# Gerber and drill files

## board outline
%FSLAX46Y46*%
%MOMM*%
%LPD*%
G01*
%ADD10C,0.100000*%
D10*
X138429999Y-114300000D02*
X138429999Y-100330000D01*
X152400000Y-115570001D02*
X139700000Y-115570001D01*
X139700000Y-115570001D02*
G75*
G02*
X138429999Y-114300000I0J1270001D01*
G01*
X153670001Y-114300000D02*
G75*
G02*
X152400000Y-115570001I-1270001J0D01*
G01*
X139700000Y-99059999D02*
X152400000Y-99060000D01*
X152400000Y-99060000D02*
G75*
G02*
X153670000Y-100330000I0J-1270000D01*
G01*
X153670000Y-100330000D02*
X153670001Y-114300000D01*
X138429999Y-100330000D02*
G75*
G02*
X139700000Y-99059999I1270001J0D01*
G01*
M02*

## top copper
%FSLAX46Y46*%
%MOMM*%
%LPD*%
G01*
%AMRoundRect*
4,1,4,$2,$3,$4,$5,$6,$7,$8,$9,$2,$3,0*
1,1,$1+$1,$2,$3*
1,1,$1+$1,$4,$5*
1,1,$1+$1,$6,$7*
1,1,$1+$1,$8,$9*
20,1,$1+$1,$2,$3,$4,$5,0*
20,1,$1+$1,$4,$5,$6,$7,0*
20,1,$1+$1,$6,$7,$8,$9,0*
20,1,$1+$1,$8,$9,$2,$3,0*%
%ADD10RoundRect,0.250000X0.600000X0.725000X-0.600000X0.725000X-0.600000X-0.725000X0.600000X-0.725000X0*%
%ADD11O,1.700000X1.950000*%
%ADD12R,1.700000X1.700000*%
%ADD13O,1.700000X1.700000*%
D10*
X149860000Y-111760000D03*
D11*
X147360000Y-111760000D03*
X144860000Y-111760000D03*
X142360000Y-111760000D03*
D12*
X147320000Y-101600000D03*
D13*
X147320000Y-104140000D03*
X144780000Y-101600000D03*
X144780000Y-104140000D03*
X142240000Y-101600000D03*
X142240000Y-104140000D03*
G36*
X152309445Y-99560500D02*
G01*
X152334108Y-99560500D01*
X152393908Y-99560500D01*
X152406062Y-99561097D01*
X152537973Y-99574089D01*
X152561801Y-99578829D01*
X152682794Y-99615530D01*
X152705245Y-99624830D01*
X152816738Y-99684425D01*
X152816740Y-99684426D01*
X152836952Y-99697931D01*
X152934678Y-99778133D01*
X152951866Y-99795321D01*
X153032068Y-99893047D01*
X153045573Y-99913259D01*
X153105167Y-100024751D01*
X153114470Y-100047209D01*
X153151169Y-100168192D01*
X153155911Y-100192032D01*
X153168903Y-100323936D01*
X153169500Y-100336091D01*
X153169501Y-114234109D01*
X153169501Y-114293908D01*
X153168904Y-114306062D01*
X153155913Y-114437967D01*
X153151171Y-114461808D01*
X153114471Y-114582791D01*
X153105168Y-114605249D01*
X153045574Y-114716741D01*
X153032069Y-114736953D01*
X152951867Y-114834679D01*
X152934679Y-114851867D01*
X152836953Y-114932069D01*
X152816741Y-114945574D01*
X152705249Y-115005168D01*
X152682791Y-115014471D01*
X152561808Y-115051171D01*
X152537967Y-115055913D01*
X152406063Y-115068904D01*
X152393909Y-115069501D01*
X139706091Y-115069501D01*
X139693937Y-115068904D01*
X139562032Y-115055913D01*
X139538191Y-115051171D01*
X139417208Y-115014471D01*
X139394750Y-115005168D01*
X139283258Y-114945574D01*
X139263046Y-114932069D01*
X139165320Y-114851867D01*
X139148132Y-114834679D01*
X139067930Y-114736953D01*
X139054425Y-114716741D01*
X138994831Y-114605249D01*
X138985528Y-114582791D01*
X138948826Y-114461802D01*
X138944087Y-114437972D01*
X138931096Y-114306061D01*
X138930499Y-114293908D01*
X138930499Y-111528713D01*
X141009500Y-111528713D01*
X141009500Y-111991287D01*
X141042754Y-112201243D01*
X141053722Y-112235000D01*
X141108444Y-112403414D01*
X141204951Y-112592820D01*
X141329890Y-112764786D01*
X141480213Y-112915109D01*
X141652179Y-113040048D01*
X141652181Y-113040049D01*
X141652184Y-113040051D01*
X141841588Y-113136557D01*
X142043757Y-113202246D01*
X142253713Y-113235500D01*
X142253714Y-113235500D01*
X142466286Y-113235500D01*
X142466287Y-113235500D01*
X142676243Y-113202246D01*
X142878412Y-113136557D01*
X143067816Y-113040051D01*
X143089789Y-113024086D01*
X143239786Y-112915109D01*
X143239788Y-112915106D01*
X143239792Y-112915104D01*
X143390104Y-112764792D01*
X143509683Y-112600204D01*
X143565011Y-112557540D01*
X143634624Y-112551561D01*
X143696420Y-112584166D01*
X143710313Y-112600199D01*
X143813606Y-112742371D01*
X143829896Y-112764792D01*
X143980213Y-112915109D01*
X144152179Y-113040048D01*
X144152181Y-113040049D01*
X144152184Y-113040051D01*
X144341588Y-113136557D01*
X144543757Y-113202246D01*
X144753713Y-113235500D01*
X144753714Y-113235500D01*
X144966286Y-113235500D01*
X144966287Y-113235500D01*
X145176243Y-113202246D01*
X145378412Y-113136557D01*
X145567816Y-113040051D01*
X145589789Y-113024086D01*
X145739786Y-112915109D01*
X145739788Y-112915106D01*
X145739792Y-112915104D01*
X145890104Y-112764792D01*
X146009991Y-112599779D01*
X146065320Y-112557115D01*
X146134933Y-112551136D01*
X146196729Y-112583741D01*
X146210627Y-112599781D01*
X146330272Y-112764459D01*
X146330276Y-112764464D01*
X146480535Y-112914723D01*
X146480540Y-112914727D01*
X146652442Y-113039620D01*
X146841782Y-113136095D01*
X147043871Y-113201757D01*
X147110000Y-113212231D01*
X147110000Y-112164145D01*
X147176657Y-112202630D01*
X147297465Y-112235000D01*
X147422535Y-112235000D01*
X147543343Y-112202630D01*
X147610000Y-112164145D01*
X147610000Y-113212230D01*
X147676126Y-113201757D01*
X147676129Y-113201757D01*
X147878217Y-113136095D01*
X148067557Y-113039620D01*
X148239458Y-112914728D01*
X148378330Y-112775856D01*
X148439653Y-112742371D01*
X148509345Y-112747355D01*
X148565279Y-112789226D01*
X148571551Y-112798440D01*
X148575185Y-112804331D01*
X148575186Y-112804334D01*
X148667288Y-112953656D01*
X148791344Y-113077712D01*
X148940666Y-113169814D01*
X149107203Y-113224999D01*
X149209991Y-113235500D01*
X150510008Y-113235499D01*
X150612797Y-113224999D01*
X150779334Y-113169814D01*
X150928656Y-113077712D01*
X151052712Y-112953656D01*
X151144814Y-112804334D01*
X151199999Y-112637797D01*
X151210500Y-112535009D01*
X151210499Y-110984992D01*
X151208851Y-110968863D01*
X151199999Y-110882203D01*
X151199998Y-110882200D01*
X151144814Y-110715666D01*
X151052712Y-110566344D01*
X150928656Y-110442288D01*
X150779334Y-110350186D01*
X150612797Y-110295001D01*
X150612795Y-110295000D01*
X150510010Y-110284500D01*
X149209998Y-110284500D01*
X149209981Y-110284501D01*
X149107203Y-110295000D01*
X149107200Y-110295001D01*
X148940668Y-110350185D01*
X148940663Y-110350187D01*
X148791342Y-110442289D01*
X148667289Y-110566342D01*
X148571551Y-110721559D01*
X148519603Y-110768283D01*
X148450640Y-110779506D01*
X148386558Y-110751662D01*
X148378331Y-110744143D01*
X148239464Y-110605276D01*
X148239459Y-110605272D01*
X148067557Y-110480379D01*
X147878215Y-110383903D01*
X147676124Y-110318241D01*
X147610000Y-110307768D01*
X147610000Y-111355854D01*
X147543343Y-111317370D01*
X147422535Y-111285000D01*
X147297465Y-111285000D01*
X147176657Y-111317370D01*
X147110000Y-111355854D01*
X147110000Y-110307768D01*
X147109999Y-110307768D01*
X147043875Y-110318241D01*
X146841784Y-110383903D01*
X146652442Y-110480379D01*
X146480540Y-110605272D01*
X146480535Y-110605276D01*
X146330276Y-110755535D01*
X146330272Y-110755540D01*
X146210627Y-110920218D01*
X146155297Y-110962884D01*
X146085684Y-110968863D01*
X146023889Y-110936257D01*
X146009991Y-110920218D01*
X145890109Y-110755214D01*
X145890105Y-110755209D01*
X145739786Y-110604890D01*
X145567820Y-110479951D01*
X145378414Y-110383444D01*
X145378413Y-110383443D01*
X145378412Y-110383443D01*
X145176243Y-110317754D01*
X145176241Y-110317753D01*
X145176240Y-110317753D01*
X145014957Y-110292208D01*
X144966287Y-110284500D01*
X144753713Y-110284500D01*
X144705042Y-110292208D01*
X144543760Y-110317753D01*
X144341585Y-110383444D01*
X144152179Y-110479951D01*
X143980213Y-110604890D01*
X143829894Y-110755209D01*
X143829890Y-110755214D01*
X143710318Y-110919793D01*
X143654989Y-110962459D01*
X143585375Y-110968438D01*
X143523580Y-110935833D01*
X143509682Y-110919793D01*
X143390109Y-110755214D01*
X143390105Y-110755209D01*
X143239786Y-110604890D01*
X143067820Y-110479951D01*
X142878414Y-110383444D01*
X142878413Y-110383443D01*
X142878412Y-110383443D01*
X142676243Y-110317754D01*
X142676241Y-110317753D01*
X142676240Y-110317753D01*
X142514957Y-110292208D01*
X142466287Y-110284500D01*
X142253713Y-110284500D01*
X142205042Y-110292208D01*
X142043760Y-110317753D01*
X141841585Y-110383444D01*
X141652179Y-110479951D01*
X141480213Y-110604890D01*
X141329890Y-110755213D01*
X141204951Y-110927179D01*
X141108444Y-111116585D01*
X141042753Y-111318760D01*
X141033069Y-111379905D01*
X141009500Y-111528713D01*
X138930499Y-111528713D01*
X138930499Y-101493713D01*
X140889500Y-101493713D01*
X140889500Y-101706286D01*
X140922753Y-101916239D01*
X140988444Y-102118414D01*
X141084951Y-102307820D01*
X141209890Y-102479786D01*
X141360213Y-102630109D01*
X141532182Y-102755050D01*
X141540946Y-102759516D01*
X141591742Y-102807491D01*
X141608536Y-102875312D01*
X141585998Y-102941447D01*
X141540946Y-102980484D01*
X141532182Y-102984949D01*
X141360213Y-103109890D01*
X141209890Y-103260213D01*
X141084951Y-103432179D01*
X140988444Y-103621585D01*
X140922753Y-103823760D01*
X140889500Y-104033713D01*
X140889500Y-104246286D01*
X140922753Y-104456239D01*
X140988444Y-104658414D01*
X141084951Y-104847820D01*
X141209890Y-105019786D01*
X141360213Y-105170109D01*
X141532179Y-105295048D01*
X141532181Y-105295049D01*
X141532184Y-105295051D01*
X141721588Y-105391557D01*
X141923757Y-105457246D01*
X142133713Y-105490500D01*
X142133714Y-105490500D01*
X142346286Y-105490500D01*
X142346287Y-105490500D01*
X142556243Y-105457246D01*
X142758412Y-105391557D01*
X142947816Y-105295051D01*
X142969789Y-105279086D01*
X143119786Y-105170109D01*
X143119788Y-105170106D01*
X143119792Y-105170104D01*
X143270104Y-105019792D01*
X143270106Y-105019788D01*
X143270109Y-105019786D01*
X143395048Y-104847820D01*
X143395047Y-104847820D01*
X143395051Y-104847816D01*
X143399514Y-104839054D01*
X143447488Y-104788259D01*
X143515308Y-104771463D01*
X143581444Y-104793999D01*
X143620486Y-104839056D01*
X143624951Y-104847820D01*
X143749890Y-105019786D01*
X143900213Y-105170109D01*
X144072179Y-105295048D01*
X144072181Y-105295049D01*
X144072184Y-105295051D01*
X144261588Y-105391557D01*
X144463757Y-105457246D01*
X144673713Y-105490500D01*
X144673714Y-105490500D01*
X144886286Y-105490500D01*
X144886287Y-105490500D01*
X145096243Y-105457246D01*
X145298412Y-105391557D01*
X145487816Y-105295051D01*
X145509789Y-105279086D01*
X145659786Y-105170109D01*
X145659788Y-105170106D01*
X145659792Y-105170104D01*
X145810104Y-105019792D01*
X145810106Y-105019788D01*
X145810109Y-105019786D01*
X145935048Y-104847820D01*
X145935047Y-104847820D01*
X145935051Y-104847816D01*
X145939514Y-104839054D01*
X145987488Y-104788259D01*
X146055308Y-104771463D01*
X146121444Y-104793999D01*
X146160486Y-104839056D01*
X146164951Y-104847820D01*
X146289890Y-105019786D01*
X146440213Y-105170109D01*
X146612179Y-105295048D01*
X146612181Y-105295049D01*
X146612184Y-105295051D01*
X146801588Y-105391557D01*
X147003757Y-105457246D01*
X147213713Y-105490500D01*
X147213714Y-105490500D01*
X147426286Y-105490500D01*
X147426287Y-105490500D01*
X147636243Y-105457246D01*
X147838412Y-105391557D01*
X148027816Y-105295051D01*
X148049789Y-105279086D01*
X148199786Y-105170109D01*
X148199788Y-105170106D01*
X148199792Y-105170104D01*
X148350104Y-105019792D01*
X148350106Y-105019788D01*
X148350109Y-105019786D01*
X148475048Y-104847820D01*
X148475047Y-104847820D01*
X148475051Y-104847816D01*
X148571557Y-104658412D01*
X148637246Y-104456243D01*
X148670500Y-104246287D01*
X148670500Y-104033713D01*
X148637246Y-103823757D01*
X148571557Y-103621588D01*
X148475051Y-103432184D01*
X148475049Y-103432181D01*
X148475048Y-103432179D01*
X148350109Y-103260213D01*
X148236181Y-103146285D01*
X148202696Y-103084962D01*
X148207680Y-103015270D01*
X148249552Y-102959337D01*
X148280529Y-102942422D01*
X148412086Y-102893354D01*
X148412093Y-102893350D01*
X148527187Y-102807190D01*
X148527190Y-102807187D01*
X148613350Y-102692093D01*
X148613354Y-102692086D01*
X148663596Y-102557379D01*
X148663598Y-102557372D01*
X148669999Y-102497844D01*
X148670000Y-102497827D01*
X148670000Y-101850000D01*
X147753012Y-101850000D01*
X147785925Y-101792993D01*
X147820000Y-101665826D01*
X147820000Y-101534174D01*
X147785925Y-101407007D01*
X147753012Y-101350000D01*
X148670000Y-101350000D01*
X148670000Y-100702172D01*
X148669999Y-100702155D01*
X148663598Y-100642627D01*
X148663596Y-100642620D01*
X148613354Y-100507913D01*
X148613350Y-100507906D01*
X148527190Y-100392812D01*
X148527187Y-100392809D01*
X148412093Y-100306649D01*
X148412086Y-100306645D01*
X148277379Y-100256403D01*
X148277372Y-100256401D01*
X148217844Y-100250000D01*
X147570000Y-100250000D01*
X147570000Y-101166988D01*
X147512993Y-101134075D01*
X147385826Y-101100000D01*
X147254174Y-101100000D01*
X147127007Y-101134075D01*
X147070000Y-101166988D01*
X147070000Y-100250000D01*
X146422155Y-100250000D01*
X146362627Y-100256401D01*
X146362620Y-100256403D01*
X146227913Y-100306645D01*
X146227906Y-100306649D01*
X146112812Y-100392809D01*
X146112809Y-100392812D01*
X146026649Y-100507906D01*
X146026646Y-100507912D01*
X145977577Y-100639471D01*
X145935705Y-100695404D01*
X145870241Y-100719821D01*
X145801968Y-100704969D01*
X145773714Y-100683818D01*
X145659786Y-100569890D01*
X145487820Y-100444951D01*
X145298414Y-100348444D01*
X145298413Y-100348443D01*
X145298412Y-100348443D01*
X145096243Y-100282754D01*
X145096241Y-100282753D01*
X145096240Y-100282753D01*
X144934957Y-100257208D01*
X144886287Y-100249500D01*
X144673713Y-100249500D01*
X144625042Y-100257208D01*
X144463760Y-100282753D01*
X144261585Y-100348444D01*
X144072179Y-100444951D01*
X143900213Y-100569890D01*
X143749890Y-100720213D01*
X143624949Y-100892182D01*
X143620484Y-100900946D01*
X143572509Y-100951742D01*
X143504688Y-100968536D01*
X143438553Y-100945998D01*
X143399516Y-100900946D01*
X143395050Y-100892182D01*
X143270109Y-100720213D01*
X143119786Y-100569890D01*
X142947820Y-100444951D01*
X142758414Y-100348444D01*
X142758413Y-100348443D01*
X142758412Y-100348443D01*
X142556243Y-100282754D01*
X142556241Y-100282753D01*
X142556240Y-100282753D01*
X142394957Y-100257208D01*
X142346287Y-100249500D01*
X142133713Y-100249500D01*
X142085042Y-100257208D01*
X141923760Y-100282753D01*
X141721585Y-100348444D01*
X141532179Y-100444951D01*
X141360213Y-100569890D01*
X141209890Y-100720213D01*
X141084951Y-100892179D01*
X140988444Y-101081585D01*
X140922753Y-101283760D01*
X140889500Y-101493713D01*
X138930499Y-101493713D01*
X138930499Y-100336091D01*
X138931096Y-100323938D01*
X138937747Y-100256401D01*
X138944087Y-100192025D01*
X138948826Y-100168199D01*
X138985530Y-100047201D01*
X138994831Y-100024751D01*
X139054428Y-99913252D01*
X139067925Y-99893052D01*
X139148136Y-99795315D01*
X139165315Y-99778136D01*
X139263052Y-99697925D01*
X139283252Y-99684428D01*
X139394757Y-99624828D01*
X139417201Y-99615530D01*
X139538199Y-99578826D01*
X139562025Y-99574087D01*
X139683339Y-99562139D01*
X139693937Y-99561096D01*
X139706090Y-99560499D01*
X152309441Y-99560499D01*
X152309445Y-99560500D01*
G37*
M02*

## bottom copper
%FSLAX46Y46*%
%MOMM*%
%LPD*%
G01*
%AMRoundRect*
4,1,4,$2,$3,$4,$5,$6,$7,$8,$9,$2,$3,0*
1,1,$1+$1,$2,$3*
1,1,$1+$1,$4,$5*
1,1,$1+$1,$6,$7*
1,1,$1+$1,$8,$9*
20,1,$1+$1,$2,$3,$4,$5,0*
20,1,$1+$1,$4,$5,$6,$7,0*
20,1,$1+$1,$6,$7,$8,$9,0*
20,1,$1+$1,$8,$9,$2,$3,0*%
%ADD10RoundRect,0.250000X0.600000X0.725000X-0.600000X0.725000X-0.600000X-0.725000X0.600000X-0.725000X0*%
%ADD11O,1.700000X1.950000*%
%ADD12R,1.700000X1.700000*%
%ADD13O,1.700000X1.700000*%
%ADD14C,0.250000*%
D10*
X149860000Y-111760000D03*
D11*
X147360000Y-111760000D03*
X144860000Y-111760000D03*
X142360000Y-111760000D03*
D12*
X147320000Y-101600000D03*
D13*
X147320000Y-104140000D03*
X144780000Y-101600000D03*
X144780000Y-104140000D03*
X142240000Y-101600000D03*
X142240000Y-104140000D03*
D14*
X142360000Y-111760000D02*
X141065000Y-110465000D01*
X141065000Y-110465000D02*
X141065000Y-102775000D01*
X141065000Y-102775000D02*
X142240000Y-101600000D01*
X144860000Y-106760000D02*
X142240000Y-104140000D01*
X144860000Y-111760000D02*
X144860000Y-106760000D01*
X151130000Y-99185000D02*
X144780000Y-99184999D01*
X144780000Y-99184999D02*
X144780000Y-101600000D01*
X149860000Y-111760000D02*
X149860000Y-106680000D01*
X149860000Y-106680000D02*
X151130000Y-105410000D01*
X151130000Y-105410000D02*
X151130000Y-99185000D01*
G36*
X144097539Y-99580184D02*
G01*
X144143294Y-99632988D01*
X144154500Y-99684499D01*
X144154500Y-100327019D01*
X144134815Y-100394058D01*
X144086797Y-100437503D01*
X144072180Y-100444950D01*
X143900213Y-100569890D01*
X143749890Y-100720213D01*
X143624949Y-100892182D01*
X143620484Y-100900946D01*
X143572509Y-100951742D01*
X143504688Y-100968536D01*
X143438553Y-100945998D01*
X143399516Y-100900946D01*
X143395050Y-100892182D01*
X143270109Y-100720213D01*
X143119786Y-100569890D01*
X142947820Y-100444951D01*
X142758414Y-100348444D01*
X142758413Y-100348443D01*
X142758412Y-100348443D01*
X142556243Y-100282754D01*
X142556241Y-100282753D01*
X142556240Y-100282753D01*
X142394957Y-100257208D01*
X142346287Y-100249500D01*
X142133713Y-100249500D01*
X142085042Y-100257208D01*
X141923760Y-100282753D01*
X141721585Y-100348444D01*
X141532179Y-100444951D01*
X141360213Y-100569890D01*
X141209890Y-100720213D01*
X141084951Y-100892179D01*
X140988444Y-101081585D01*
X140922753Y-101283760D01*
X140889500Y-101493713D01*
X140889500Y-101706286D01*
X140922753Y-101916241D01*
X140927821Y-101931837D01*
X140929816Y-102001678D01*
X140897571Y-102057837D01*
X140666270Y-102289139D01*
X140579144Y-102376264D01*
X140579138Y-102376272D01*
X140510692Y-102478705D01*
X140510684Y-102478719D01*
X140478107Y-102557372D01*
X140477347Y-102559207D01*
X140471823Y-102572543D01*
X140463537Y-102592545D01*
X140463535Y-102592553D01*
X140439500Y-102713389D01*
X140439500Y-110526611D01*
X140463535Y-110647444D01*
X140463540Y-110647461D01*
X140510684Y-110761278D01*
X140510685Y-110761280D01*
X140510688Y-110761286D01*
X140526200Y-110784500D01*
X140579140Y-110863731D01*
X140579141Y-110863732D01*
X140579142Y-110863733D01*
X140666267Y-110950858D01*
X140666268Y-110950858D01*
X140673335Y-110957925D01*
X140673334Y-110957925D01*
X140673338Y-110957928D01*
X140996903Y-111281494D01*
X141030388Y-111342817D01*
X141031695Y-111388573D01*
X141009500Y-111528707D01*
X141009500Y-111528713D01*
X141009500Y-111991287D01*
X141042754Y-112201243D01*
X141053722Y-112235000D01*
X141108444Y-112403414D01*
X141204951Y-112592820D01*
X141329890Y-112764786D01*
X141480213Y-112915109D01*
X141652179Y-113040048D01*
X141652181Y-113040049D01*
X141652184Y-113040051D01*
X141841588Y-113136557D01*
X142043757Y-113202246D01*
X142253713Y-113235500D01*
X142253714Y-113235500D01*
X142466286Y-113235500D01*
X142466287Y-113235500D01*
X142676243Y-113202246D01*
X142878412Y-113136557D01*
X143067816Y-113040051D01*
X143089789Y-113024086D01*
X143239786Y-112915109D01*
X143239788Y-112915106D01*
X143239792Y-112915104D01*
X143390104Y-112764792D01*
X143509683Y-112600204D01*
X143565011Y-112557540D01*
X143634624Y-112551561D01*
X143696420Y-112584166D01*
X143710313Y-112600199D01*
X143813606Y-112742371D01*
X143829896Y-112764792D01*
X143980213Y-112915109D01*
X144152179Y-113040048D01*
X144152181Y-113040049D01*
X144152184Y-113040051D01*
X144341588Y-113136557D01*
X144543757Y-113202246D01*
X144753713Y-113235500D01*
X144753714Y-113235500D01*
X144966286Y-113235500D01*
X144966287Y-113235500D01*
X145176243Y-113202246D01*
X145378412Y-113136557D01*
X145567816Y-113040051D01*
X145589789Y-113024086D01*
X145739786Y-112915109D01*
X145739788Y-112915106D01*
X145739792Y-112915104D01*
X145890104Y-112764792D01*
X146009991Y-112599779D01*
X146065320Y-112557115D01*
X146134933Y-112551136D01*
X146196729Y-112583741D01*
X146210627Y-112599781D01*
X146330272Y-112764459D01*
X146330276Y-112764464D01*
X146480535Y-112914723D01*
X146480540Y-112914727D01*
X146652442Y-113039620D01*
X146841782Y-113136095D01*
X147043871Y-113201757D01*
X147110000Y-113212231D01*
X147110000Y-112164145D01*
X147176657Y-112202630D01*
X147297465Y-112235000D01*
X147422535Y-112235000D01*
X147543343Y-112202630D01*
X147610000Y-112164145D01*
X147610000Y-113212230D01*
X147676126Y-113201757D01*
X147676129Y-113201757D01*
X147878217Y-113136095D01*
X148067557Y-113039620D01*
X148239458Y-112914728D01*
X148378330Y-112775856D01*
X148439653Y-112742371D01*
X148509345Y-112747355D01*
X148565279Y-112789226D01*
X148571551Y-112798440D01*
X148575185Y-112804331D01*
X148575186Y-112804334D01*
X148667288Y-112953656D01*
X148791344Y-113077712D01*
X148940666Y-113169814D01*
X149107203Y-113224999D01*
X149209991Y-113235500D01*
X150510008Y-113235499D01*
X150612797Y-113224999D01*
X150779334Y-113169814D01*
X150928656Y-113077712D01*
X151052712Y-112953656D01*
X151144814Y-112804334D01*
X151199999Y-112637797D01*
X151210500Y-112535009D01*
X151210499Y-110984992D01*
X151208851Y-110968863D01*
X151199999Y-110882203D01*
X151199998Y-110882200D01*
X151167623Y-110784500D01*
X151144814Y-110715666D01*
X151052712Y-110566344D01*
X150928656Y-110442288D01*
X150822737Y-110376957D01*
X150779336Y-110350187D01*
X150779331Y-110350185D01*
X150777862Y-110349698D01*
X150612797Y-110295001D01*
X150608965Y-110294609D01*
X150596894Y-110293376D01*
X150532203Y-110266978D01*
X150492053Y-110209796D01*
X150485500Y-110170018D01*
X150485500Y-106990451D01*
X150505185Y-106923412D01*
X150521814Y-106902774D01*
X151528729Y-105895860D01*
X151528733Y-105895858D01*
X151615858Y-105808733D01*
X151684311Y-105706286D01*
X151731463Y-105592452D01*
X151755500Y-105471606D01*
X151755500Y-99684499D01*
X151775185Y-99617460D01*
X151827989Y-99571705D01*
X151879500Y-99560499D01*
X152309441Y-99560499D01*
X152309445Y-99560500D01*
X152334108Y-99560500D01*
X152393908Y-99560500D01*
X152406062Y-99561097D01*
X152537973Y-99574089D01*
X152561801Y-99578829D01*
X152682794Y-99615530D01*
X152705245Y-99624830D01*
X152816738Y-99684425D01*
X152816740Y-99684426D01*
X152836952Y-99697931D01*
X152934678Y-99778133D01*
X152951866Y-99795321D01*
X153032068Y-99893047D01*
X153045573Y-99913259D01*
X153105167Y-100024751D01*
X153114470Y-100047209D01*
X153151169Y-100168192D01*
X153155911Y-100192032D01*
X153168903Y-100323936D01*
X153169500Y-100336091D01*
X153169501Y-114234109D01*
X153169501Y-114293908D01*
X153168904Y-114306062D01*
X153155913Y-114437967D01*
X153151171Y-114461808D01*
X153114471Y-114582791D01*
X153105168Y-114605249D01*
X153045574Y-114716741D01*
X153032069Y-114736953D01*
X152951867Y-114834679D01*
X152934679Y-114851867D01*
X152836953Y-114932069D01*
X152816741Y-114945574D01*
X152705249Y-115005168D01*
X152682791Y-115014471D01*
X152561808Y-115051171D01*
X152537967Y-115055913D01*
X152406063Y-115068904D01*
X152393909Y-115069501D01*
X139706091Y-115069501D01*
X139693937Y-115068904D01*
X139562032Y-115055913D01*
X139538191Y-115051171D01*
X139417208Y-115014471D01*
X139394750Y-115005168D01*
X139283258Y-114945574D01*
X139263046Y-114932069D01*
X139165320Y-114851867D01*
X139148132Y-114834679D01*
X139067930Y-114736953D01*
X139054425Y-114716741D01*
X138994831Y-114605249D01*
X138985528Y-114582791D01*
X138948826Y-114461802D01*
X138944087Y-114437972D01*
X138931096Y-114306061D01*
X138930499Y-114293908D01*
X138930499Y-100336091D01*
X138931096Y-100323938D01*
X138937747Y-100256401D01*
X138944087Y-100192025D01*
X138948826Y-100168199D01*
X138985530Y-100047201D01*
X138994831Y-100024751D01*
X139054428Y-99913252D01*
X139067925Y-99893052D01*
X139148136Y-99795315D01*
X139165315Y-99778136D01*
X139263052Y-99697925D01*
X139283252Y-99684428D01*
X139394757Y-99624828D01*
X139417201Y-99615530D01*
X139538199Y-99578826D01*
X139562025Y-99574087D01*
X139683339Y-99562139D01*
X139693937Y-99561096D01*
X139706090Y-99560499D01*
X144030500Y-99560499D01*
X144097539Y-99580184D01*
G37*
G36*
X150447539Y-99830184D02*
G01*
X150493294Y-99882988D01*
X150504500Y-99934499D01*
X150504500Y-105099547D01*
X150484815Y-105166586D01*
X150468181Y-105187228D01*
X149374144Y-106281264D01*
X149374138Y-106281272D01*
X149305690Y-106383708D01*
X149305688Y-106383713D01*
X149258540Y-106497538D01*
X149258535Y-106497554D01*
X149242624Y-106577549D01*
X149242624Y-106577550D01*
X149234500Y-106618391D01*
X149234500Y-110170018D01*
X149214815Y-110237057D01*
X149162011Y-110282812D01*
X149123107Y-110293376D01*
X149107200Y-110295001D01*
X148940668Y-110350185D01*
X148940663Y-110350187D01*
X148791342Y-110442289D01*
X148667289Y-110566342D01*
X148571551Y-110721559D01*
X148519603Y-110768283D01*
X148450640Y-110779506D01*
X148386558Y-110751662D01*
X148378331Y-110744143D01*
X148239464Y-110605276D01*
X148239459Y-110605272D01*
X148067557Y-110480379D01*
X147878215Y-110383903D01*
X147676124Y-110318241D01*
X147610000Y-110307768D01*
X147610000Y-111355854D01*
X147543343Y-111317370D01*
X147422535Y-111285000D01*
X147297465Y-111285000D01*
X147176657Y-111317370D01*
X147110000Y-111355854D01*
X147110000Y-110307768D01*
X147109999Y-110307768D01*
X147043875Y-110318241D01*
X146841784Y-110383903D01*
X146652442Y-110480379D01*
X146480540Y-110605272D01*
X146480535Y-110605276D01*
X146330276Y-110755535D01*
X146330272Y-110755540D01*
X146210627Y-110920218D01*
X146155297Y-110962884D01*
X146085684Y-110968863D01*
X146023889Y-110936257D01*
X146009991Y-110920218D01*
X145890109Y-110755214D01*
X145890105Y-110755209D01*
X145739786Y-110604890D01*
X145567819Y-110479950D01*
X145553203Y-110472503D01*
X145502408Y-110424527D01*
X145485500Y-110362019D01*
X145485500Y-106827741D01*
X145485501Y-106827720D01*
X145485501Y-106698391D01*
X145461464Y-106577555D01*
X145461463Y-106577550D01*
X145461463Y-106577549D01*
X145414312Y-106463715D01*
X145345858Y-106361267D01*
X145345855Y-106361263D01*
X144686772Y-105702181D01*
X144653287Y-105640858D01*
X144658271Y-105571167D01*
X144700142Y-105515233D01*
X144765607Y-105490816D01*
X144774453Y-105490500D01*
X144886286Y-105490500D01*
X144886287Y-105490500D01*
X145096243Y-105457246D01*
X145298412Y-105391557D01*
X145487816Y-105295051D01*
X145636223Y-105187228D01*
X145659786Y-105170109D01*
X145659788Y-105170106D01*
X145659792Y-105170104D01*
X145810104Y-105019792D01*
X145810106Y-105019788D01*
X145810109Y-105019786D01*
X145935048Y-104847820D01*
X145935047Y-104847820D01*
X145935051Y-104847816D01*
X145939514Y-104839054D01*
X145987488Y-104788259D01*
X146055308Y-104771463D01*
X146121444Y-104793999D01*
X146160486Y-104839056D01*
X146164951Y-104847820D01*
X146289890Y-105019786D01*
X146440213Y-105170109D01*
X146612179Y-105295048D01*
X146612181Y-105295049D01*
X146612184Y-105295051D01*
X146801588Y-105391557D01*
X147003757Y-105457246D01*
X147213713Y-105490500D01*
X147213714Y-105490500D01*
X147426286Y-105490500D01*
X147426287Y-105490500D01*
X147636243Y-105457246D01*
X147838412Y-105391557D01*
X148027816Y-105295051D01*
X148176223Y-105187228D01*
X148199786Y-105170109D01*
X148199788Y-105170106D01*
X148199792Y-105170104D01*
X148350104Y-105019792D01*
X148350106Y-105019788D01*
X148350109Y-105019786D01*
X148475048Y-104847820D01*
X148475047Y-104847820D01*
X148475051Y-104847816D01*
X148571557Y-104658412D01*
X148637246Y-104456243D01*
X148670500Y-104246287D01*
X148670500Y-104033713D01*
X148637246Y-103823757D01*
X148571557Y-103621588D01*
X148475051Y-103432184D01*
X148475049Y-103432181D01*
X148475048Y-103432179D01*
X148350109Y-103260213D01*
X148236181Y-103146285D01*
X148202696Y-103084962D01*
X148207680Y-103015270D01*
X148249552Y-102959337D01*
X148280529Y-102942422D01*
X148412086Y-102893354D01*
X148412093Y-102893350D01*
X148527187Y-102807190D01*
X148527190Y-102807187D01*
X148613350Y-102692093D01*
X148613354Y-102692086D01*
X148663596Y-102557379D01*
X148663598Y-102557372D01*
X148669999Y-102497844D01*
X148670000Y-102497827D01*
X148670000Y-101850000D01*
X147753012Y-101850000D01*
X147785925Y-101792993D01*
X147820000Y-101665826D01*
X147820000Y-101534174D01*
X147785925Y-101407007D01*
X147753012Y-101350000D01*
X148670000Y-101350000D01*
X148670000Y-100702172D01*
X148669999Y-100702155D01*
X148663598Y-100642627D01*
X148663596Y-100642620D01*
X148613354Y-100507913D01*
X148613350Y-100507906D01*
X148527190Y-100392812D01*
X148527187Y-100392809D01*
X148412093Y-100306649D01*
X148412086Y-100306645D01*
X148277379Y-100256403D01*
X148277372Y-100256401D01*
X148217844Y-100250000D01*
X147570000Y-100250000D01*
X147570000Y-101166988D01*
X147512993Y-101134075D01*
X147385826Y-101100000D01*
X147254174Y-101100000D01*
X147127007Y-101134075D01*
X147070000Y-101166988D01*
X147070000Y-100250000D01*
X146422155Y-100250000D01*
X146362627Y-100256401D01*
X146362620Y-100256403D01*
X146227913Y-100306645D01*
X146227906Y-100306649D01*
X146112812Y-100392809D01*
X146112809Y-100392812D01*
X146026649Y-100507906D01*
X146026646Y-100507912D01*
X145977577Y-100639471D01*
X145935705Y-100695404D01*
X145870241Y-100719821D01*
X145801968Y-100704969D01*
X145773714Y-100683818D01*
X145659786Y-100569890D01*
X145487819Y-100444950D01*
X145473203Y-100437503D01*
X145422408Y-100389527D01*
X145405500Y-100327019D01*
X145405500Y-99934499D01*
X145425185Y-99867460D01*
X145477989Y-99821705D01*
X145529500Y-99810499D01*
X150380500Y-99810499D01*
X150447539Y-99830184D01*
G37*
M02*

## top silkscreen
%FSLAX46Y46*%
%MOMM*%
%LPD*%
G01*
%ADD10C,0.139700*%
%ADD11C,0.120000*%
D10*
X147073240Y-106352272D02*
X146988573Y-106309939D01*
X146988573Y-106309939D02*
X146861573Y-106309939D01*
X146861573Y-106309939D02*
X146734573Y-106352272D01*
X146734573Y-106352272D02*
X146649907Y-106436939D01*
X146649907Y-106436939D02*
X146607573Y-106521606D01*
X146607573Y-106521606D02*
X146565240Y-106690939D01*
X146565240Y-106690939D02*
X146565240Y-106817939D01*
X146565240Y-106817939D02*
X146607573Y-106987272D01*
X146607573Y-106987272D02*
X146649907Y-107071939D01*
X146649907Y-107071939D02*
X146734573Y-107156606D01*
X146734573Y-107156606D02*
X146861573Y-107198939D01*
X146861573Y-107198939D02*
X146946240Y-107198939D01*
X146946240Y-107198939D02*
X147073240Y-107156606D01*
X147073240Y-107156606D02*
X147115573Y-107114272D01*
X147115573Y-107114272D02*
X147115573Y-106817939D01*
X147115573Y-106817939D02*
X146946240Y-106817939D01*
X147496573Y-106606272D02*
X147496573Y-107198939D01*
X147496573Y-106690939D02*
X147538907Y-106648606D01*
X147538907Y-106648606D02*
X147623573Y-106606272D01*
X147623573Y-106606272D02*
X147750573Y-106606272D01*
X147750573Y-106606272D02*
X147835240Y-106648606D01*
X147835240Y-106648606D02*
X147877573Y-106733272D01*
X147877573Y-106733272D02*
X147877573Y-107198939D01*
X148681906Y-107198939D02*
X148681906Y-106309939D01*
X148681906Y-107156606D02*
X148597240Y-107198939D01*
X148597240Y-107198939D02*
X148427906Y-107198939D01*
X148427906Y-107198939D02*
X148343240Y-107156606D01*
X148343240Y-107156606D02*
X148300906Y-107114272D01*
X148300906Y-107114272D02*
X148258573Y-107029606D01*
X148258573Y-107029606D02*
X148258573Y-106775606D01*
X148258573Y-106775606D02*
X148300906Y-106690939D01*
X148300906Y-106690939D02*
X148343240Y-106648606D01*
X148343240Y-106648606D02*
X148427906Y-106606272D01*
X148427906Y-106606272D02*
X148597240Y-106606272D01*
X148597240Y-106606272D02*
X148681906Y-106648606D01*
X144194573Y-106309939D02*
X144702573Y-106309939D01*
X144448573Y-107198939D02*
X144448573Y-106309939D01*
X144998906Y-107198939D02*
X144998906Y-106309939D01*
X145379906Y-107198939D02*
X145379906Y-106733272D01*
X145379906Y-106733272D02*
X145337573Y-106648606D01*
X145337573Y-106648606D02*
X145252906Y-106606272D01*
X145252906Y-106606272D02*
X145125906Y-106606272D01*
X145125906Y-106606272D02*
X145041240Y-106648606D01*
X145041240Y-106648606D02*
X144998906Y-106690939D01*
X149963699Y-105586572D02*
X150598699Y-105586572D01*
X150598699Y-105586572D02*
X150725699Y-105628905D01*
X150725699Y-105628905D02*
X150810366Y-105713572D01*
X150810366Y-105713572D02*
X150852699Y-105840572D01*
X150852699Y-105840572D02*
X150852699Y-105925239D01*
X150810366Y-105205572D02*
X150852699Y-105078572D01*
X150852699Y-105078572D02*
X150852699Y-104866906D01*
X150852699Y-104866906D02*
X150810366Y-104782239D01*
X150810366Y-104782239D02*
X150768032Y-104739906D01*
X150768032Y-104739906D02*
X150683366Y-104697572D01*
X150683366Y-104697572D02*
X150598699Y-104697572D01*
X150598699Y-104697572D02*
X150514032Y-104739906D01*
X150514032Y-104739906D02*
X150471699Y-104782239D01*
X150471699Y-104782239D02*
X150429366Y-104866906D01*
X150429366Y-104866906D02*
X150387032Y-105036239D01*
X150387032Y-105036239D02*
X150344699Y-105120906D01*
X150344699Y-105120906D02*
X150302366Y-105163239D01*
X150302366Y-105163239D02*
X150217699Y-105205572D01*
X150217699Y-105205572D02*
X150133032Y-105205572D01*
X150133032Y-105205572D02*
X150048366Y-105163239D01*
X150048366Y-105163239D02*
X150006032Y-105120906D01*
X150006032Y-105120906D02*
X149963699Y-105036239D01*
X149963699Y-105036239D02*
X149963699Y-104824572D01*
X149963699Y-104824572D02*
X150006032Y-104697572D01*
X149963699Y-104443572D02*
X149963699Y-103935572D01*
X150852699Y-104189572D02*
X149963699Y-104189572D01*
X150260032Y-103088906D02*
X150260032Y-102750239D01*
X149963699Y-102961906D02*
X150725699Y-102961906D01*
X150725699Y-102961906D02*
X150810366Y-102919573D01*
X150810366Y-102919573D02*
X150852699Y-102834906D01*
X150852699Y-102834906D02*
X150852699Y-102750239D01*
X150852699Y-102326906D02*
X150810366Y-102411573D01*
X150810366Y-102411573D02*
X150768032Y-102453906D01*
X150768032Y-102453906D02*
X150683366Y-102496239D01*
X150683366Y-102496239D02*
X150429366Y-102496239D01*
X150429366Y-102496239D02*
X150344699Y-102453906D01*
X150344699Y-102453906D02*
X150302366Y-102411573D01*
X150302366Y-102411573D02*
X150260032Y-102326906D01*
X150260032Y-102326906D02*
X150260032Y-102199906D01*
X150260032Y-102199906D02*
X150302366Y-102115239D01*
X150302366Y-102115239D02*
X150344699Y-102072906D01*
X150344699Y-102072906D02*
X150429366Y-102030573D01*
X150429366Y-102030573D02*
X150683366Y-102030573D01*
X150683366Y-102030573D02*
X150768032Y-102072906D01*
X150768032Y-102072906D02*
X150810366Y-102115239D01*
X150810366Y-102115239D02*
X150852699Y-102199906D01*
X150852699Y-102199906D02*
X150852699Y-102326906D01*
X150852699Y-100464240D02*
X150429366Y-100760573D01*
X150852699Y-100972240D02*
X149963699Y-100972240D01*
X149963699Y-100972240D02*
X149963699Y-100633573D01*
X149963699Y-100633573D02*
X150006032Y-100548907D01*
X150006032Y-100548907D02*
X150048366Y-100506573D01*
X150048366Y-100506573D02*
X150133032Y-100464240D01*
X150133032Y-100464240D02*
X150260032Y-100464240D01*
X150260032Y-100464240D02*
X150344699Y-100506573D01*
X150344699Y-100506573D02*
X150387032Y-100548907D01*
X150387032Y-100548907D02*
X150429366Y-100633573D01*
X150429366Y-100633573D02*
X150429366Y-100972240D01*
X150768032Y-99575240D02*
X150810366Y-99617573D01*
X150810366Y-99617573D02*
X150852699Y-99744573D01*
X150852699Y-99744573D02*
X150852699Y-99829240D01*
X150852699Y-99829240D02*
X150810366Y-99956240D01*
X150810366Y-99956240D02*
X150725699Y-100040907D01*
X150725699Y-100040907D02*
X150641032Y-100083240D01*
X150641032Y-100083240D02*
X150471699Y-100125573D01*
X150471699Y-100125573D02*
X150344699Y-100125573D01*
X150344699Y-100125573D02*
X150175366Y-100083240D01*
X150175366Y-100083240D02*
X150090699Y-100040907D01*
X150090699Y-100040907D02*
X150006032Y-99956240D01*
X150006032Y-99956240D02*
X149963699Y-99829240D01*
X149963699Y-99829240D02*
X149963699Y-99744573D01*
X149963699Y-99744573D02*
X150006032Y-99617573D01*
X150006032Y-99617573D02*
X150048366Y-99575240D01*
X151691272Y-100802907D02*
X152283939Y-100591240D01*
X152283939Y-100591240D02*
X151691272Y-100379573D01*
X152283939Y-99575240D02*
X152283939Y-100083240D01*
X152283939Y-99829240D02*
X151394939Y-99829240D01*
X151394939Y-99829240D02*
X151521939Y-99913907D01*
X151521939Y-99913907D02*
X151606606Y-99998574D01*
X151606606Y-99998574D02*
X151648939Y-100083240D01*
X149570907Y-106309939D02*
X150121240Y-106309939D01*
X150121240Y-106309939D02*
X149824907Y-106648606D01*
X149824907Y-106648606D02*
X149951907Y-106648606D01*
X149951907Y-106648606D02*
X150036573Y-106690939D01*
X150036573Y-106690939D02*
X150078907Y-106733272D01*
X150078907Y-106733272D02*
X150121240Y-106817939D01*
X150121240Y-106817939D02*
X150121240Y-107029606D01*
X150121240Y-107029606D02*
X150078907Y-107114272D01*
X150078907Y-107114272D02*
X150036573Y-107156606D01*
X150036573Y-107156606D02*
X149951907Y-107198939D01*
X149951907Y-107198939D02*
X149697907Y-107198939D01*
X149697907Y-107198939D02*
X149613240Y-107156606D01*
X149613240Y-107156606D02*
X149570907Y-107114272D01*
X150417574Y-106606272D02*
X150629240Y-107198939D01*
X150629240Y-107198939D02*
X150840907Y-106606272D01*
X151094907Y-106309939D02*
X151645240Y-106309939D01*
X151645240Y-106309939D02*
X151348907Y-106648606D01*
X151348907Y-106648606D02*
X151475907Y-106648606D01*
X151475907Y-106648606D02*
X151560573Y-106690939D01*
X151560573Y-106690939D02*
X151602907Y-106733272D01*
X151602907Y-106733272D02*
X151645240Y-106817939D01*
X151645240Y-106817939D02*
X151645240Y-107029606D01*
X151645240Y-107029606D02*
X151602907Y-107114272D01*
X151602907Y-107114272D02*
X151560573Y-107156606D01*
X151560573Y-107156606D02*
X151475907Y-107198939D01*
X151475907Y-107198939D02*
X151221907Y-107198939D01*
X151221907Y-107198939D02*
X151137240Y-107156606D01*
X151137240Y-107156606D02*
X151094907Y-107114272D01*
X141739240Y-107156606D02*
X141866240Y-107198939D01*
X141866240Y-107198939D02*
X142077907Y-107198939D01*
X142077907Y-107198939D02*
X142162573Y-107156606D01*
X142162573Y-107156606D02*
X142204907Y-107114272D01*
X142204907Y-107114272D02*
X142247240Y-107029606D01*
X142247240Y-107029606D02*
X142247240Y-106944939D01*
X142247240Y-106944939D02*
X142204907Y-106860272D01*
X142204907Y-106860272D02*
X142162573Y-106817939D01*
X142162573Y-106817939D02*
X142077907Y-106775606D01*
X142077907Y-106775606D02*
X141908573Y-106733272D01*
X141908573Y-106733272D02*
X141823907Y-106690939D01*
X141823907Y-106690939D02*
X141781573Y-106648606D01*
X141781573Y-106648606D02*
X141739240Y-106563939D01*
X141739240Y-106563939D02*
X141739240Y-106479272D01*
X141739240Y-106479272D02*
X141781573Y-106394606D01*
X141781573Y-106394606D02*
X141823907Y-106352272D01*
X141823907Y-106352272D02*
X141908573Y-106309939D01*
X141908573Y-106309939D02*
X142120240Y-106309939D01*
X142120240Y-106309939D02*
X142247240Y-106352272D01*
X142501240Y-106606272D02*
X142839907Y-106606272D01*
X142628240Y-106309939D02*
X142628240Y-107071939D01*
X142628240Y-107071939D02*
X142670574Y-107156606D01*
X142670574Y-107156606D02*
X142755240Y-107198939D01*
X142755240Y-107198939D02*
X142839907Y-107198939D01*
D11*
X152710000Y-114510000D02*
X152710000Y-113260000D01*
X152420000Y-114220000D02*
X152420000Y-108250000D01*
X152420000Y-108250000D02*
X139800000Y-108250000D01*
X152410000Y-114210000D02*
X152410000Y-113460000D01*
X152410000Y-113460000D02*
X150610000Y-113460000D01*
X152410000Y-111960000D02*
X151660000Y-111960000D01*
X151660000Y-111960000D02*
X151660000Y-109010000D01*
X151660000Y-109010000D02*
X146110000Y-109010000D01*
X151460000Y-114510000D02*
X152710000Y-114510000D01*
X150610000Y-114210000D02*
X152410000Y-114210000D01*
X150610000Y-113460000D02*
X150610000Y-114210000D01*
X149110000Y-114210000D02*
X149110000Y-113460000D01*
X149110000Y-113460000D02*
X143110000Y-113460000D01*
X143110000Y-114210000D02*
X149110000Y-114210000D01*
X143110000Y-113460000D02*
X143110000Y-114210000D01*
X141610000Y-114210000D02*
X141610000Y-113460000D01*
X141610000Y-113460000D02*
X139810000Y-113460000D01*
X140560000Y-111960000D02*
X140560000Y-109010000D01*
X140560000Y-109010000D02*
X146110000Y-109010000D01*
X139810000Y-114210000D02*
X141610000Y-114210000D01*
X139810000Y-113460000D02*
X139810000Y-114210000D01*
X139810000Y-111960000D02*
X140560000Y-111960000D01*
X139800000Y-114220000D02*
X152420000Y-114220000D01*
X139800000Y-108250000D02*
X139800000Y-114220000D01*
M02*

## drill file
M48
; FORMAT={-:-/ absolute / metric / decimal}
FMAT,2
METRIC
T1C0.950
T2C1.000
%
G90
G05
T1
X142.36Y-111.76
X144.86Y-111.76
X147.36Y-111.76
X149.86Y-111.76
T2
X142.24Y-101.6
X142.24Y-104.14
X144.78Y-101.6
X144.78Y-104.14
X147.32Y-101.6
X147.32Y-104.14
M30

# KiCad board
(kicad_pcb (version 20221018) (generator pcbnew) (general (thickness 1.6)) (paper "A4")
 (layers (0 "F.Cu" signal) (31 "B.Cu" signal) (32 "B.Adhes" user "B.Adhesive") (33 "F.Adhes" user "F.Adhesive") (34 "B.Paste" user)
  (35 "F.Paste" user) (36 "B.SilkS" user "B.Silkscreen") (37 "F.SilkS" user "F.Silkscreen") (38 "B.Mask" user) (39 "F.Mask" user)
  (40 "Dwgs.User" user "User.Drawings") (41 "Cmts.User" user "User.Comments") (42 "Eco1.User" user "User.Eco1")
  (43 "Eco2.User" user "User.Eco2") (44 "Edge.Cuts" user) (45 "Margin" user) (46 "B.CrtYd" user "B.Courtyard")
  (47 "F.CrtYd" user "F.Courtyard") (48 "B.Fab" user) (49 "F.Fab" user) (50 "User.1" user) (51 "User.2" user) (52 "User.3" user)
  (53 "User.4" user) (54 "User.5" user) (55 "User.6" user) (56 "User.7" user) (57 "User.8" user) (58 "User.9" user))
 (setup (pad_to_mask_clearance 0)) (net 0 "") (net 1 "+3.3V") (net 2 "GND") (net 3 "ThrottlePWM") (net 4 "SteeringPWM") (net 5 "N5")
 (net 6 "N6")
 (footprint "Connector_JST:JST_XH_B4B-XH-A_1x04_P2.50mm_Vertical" (layer "F.Cu") (at 149.86 111.76 180)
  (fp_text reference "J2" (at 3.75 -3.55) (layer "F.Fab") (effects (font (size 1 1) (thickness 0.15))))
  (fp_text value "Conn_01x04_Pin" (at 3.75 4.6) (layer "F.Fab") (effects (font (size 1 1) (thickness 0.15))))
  (fp_line (start -2.85 -2.75) (end -2.85 -1.5) (stroke (width 0.12) (type solid)) (layer "F.SilkS"))
  (fp_line (start -2.56 -2.46) (end -2.56 3.51) (stroke (width 0.12) (type solid)) (layer "F.SilkS"))
  (fp_line (start -2.56 3.51) (end 10.06 3.51) (stroke (width 0.12) (type solid)) (layer "F.SilkS"))
  (fp_line (start -2.55 -2.45) (end -2.55 -1.7) (stroke (width 0.12) (type solid)) (layer "F.SilkS"))
  (fp_line (start -2.55 -1.7) (end -0.75 -1.7) (stroke (width 0.12) (type solid)) (layer "F.SilkS"))
  (fp_line (start -2.55 -0.2) (end -1.8 -0.2) (stroke (width 0.12) (type solid)) (layer "F.SilkS"))
  (fp_line (start -1.8 -0.2) (end -1.8 2.75) (stroke (width 0.12) (type solid)) (layer "F.SilkS"))
  (fp_line (start -1.8 2.75) (end 3.75 2.75) (stroke (width 0.12) (type solid)) (layer "F.SilkS"))
  (fp_line (start -1.6 -2.75) (end -2.85 -2.75) (stroke (width 0.12) (type solid)) (layer "F.SilkS"))
  (fp_line (start -0.75 -2.45) (end -2.55 -2.45) (stroke (width 0.12) (type solid)) (layer "F.SilkS"))
  (fp_line (start -0.75 -1.7) (end -0.75 -2.45) (stroke (width 0.12) (type solid)) (layer "F.SilkS"))
  (fp_line (start 0.75 -2.45) (end 0.75 -1.7) (stroke (width 0.12) (type solid)) (layer "F.SilkS"))
  (fp_line (start 0.75 -1.7) (end 6.75 -1.7) (stroke (width 0.12) (type solid)) (layer "F.SilkS"))
  (fp_line (start 6.75 -2.45) (end 0.75 -2.45) (stroke (width 0.12) (type solid)) (layer "F.SilkS"))
  (fp_line (start 6.75 -1.7) (end 6.75 -2.45) (stroke (width 0.12) (type solid)) (layer "F.SilkS"))
  (fp_line (start 8.25 -2.45) (end 8.25 -1.7) (stroke (width 0.12) (type solid)) (layer "F.SilkS"))
  (fp_line (start 8.25 -1.7) (end 10.05 -1.7) (stroke (width 0.12) (type solid)) (layer "F.SilkS"))
  (fp_line (start 9.3 -0.2) (end 9.3 2.75) (stroke (width 0.12) (type solid)) (layer "F.SilkS"))
  (fp_line (start 9.3 2.75) (end 3.75 2.75) (stroke (width 0.12) (type solid)) (layer "F.SilkS"))
  (fp_line (start 10.05 -2.45) (end 8.25 -2.45) (stroke (width 0.12) (type solid)) (layer "F.SilkS"))
  (fp_line (start 10.05 -1.7) (end 10.05 -2.45) (stroke (width 0.12) (type solid)) (layer "F.SilkS"))
  (fp_line (start 10.05 -0.2) (end 9.3 -0.2) (stroke (width 0.12) (type solid)) (layer "F.SilkS"))
  (fp_line (start 10.06 -2.46) (end -2.56 -2.46) (stroke (width 0.12) (type solid)) (layer "F.SilkS"))
  (fp_line (start 10.06 3.51) (end 10.06 -2.46) (stroke (width 0.12) (type solid)) (layer "F.SilkS"))
  (pad "1" thru_hole roundrect (at 0 0 180) (size 1.7 1.95) (drill 0.95) (layers "*.Cu" "*.Mask") (roundrect_rratio 0.147059)
   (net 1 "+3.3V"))
  (pad "2" thru_hole oval (at 2.5 0 180) (size 1.7 1.95) (drill 0.95) (layers "*.Cu" "*.Mask") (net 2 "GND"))
  (pad "3" thru_hole oval (at 5 0 180) (size 1.7 1.95) (drill 0.95) (layers "*.Cu" "*.Mask") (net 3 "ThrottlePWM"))
  (pad "4" thru_hole oval (at 7.5 0 180) (size 1.7 1.95) (drill 0.95) (layers "*.Cu" "*.Mask") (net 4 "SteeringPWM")))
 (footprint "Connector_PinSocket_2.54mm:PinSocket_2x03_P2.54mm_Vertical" (layer "B.Cu") (at 147.32 101.6 90)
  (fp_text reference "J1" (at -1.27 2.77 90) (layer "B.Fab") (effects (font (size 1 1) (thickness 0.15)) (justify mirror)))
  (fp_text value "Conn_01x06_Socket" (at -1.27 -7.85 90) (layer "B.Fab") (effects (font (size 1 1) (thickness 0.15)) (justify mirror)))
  (pad "1" thru_hole rect (at 0 0 90) (size 1.7 1.7) (drill 1) (layers "*.Cu" "*.Mask") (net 2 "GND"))
  (pad "2" thru_hole oval (at -2.54 0 90) (size 1.7 1.7) (drill 1) (layers "*.Cu" "*.Mask") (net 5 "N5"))
  (pad "3" thru_hole oval (at 0 -2.54 90) (size 1.7 1.7) (drill 1) (layers "*.Cu" "*.Mask") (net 1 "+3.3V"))
  (pad "4" thru_hole oval (at -2.54 -2.54 90) (size 1.7 1.7) (drill 1) (layers "*.Cu" "*.Mask") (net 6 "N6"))
  (pad "5" thru_hole oval (at 0 -5.08 90) (size 1.7 1.7) (drill 1) (layers "*.Cu" "*.Mask") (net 4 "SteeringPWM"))
  (pad "6" thru_hole oval (at -2.54 -5.08 90) (size 1.7 1.7) (drill 1) (layers "*.Cu" "*.Mask") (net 3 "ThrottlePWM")))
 (gr_line (start 138.429999 114.3) (end 138.429999 100.33) (stroke (width 0.1) (type default)) (layer "Edge.Cuts"))
 (gr_line (start 152.4 115.570001) (end 139.7 115.570001) (stroke (width 0.1) (type default)) (layer "Edge.Cuts"))
 (gr_arc (start 139.7 115.570001) (mid 138.801973 115.198027) (end 138.429999 114.3) (stroke (width 0.1) (type default)) (layer "Edge.Cuts"))
 (gr_arc (start 153.670001 114.3) (mid 153.298027 115.198027) (end 152.4 115.570001) (stroke (width 0.1) (type default)) (layer "Edge.Cuts"))
 (gr_line (start 139.7 99.059999) (end 152.4 99.06) (stroke (width 0.1) (type default)) (layer "Edge.Cuts"))
 (gr_arc (start 152.4 99.06) (mid 153.298026 99.431974) (end 153.67 100.33) (stroke (width 0.1) (type default)) (layer "Edge.Cuts"))
 (gr_line (start 153.67 100.33) (end 153.670001 114.3) (stroke (width 0.1) (type default)) (layer "Edge.Cuts"))
 (gr_arc (start 138.429999 100.33) (mid 138.801973 99.431973) (end 139.7 99.059999) (stroke (width 0.1) (type default)) (layer "Edge.Cuts"))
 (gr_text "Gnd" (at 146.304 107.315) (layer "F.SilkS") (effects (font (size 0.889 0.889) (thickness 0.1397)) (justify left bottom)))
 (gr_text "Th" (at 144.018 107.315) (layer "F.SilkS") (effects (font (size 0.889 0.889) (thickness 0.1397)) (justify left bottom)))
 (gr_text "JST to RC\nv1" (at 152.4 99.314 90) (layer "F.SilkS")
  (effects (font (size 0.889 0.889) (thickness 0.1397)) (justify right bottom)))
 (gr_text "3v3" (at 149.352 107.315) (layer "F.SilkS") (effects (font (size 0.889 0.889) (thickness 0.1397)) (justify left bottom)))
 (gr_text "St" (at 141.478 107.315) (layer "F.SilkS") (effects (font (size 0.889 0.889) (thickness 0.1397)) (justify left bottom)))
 (segment (start 142.36 111.76) (end 141.065 110.465) (width 0.25) (layer "B.Cu") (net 4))
 (segment (start 141.065 110.465) (end 141.065 102.775) (width 0.25) (layer "B.Cu") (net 4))
 (segment (start 141.065 102.775) (end 142.24 101.6) (width 0.25) (layer "B.Cu") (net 4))
 (segment (start 144.86 106.76) (end 142.24 104.14) (width 0.25) (layer "B.Cu") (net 3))
 (segment (start 144.86 111.76) (end 144.86 106.76) (width 0.25) (layer "B.Cu") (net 3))
 (segment (start 151.13 99.185) (end 144.78 99.184999) (width 0.25) (layer "B.Cu") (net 1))
 (segment (start 144.78 99.184999) (end 144.78 101.6) (width 0.25) (layer "B.Cu") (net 1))
 (segment (start 149.86 111.76) (end 149.86 106.68) (width 0.25) (layer "B.Cu") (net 1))
 (segment (start 149.86 106.68) (end 151.13 105.41) (width 0.25) (layer "B.Cu") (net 1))
 (segment (start 151.13 105.41) (end 151.13 99.185) (width 0.25) (layer "B.Cu") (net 1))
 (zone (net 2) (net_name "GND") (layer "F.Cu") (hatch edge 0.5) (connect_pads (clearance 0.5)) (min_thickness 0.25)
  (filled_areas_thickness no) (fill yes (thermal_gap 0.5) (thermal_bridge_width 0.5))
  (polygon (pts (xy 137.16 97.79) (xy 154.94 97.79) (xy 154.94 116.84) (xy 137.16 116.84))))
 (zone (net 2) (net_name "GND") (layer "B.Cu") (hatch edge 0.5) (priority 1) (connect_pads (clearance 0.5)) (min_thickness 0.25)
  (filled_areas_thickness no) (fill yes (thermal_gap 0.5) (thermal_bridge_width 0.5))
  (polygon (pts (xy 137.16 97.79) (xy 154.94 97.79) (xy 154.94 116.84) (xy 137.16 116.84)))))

